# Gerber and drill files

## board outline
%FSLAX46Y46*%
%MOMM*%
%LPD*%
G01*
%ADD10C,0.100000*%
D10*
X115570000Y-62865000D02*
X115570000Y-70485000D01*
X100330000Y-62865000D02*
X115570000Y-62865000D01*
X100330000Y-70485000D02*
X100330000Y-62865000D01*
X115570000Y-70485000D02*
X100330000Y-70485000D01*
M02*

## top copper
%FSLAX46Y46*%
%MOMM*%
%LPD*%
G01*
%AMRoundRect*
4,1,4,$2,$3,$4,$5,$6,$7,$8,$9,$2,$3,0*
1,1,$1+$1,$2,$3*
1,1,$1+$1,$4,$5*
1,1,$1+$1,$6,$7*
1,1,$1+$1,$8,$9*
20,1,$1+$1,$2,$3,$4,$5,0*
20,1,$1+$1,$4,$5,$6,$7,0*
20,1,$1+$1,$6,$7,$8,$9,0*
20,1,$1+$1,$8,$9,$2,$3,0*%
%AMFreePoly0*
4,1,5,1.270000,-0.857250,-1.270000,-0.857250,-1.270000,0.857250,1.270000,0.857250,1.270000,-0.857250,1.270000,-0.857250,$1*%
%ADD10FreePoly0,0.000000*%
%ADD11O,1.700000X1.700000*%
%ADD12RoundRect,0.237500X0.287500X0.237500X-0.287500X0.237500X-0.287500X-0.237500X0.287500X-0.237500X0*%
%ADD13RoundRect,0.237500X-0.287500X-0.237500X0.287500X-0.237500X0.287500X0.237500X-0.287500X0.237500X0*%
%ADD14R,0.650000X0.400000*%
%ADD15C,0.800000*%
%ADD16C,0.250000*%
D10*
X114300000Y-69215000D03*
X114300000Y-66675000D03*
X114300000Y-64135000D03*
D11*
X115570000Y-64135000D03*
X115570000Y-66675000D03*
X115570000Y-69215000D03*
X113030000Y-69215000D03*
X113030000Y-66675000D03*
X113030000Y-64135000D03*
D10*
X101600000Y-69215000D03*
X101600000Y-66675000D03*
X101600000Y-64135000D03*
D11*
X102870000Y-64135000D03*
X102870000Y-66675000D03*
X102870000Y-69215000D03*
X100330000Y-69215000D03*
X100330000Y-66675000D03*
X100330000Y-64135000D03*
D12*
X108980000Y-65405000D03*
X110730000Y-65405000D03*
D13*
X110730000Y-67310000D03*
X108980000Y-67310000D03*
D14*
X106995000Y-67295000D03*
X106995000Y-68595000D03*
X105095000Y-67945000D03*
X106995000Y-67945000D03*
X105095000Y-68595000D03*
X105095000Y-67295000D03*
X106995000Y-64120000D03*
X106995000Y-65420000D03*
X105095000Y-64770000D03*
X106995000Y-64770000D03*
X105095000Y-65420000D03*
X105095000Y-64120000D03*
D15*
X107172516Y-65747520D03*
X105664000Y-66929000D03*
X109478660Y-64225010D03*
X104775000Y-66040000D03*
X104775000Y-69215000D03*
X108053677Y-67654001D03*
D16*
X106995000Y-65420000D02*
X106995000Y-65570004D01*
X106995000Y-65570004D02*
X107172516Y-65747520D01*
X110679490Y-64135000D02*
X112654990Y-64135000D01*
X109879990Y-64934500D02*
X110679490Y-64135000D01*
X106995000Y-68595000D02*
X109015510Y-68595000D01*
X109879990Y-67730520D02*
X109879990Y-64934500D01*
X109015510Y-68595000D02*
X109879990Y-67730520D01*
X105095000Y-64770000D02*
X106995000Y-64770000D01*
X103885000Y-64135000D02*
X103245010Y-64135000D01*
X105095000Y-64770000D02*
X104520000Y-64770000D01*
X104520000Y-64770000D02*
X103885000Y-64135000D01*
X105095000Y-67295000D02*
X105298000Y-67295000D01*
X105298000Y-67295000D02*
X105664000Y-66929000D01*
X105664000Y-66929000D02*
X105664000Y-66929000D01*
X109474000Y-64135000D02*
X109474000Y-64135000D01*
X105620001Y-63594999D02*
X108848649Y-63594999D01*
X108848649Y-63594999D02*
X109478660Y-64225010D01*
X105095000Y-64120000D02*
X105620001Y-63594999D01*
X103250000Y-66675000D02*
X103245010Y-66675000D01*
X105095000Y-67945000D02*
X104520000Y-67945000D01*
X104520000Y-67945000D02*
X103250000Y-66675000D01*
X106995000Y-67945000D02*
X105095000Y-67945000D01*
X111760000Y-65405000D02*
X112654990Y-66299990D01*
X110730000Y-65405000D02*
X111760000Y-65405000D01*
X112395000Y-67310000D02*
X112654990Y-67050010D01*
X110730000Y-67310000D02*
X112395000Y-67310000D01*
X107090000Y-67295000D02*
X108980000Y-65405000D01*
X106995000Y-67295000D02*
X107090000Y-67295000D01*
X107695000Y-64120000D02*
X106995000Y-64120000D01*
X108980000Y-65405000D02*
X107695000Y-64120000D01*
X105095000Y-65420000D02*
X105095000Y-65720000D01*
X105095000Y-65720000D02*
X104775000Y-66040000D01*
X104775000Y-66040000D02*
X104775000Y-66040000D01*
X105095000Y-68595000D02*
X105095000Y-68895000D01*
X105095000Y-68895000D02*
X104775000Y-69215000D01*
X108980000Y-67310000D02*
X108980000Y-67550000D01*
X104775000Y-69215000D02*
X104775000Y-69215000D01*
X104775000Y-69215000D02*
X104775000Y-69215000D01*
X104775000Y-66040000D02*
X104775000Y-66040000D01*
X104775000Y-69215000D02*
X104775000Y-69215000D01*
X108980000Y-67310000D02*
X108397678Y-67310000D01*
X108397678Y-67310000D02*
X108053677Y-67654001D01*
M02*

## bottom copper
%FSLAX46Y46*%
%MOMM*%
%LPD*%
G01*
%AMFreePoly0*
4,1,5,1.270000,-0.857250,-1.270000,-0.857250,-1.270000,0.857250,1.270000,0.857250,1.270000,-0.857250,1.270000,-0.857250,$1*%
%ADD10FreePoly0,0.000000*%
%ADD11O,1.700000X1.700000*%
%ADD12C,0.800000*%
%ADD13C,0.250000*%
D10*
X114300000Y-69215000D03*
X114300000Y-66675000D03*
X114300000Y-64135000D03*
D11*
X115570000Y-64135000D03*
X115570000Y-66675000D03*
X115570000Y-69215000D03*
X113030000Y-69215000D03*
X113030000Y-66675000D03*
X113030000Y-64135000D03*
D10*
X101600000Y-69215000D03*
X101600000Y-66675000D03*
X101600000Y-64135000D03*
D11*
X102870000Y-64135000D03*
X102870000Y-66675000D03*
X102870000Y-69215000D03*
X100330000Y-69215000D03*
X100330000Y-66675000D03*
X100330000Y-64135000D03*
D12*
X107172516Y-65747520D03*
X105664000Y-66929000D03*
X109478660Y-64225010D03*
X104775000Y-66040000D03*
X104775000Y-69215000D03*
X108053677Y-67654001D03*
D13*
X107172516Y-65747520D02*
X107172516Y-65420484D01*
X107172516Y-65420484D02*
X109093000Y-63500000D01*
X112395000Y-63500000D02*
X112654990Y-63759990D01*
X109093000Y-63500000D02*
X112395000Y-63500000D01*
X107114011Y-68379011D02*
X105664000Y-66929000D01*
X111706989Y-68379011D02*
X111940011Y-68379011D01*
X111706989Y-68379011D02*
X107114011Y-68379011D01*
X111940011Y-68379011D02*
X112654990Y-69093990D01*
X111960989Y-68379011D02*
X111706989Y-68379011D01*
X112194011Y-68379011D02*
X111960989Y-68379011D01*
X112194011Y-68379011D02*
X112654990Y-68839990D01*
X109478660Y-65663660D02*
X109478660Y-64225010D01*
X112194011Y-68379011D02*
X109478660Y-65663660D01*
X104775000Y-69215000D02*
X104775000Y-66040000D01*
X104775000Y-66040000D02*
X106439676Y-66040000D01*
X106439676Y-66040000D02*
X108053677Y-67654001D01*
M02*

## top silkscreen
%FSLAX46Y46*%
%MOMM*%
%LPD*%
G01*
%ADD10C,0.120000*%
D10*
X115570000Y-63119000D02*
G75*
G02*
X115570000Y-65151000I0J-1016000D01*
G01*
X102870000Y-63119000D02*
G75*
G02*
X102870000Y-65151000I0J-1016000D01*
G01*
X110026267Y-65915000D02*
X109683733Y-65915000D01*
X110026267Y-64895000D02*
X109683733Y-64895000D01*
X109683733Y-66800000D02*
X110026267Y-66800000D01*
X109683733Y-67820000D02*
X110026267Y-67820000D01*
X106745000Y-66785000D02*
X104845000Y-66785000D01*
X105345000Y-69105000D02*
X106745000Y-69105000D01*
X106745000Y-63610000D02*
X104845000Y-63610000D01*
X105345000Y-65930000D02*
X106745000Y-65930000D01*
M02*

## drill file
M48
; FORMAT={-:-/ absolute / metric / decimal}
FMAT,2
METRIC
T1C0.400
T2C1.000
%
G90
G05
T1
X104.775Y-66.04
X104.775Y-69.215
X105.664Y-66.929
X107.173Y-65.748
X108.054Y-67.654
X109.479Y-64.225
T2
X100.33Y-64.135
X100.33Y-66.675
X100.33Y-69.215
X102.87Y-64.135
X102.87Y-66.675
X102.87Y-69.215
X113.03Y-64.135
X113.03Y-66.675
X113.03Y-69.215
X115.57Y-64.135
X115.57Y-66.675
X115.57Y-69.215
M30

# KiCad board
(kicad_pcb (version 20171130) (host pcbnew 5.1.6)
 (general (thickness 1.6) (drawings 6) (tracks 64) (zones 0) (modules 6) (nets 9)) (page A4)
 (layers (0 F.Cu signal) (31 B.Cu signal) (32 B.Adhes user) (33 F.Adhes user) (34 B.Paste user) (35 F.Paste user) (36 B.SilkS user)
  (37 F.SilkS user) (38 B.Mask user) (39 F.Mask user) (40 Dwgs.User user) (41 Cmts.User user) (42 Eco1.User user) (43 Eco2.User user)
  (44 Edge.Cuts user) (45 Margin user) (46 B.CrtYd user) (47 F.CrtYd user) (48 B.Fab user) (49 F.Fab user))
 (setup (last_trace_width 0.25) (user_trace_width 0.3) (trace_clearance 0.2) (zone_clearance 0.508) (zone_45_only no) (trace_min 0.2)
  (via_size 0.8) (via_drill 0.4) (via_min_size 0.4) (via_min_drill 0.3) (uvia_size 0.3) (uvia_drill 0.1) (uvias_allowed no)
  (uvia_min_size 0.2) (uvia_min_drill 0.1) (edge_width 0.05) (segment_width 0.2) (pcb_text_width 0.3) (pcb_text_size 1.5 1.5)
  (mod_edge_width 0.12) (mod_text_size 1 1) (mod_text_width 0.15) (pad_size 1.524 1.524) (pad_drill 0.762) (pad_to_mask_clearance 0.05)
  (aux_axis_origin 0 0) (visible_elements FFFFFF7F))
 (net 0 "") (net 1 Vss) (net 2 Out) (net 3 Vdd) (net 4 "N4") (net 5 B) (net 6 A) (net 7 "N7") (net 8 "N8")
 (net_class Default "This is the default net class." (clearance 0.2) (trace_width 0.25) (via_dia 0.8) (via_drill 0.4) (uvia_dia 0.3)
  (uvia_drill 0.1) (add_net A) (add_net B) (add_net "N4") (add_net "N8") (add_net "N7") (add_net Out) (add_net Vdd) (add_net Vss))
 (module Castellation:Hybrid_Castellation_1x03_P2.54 (layer F.Cu) (at 114.3 64.135)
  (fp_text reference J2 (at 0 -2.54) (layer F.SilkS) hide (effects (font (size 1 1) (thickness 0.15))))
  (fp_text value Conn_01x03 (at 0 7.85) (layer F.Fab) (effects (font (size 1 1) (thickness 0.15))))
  (fp_arc (start 1.27 0) (end 1.27 1.016) (angle -180) (layer F.SilkS) (width 0.12))
  (pad 3 connect custom (at 0 5.08) (size 2.54 1.7145) (layers B.Cu B.Mask) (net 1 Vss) (zone_connect 0)
   (options (clearance outline) (anchor rect)) (primitives))
  (pad 2 connect custom (at 0 2.54) (size 2.54 1.7145) (layers B.Cu B.Mask) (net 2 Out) (zone_connect 0)
   (options (clearance outline) (anchor rect)) (primitives))
  (pad 1 connect custom (at 0 0) (size 2.54 1.7145) (layers B.Cu B.Mask) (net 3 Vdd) (zone_connect 0)
   (options (clearance outline) (anchor rect)) (primitives))
  (pad 3 connect custom (at 0 5.08) (size 2.54 1.7145) (layers F.Cu F.Mask) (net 1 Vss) (zone_connect 0)
   (options (clearance outline) (anchor rect)) (primitives))
  (pad 2 connect custom (at 0 2.54) (size 2.54 1.7145) (layers F.Cu F.Mask) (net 2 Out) (zone_connect 0)
   (options (clearance outline) (anchor rect)) (primitives))
  (pad 1 connect custom (at 0 0) (size 2.54 1.7145) (layers F.Cu F.Mask) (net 3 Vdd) (zone_connect 0)
   (options (clearance outline) (anchor rect)) (primitives))
  (pad 1 thru_hole oval (at 1.27 0) (size 1.7 1.7) (drill 1) (layers *.Cu *.Mask) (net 3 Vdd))
  (pad 2 thru_hole oval (at 1.27 2.54) (size 1.7 1.7) (drill 1) (layers *.Cu *.Mask) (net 2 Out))
  (pad 3 thru_hole oval (at 1.27 5.08) (size 1.7 1.7) (drill 1) (layers *.Cu *.Mask) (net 1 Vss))
  (pad 3 thru_hole oval (at -1.27 5.08) (size 1.7 1.7) (drill 1) (layers *.Cu *.Mask) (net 1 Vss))
  (pad 2 thru_hole oval (at -1.27 2.54) (size 1.7 1.7) (drill 1) (layers *.Cu *.Mask) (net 2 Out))
  (pad 1 thru_hole oval (at -1.27 0) (size 1.7 1.7) (drill 1) (layers *.Cu *.Mask) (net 3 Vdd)))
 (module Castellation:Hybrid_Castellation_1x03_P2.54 (layer F.Cu) (at 101.6 64.135)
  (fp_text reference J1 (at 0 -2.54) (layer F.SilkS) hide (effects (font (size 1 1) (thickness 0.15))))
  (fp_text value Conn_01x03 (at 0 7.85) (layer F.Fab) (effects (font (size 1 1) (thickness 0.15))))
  (fp_arc (start 1.27 0) (end 1.27 1.016) (angle -180) (layer F.SilkS) (width 0.12))
  (pad 3 connect custom (at 0 5.08) (size 2.54 1.7145) (layers B.Cu B.Mask) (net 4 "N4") (zone_connect 0)
   (options (clearance outline) (anchor rect)) (primitives))
  (pad 2 connect custom (at 0 2.54) (size 2.54 1.7145) (layers B.Cu B.Mask) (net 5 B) (zone_connect 0)
   (options (clearance outline) (anchor rect)) (primitives))
  (pad 1 connect custom (at 0 0) (size 2.54 1.7145) (layers B.Cu B.Mask) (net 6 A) (zone_connect 0)
   (options (clearance outline) (anchor rect)) (primitives))
  (pad 3 connect custom (at 0 5.08) (size 2.54 1.7145) (layers F.Cu F.Mask) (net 4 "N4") (zone_connect 0)
   (options (clearance outline) (anchor rect)) (primitives))
  (pad 2 connect custom (at 0 2.54) (size 2.54 1.7145) (layers F.Cu F.Mask) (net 5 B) (zone_connect 0)
   (options (clearance outline) (anchor rect)) (primitives))
  (pad 1 connect custom (at 0 0) (size 2.54 1.7145) (layers F.Cu F.Mask) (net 6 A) (zone_connect 0)
   (options (clearance outline) (anchor rect)) (primitives))
  (pad 1 thru_hole oval (at 1.27 0) (size 1.7 1.7) (drill 1) (layers *.Cu *.Mask) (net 6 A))
  (pad 2 thru_hole oval (at 1.27 2.54) (size 1.7 1.7) (drill 1) (layers *.Cu *.Mask) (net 5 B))
  (pad 3 thru_hole oval (at 1.27 5.08) (size 1.7 1.7) (drill 1) (layers *.Cu *.Mask) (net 4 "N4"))
  (pad 3 thru_hole oval (at -1.27 5.08) (size 1.7 1.7) (drill 1) (layers *.Cu *.Mask) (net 4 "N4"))
  (pad 2 thru_hole oval (at -1.27 2.54) (size 1.7 1.7) (drill 1) (layers *.Cu *.Mask) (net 5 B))
  (pad 1 thru_hole oval (at -1.27 0) (size 1.7 1.7) (drill 1) (layers *.Cu *.Mask) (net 6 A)))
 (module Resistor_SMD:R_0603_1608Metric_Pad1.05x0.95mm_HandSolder (layer F.Cu) (at 109.855 65.405 180)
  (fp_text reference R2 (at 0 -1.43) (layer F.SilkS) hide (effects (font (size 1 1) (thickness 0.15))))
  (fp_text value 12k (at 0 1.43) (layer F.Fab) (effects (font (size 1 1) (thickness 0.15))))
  (fp_line (start -0.171267 -0.51) (end 0.171267 -0.51) (layer F.SilkS) (width 0.12))
  (fp_line (start -0.171267 0.51) (end 0.171267 0.51) (layer F.SilkS) (width 0.12))
  (pad 2 smd roundrect (at 0.875 0 180) (size 1.05 0.95) (layers F.Cu F.Paste F.Mask) (roundrect_rratio 0.25) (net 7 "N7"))
  (pad 1 smd roundrect (at -0.875 0 180) (size 1.05 0.95) (layers F.Cu F.Paste F.Mask) (roundrect_rratio 0.25) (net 2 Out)))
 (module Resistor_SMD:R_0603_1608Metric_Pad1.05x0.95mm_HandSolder (layer F.Cu) (at 109.855 67.31)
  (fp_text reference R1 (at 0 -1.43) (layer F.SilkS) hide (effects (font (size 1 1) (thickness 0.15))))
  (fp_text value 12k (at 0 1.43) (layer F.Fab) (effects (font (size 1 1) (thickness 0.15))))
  (fp_line (start -0.171267 -0.51) (end 0.171267 -0.51) (layer F.SilkS) (width 0.12))
  (fp_line (start -0.171267 0.51) (end 0.171267 0.51) (layer F.SilkS) (width 0.12))
  (pad 2 smd roundrect (at 0.875 0) (size 1.05 0.95) (layers F.Cu F.Paste F.Mask) (roundrect_rratio 0.25) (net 2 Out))
  (pad 1 smd roundrect (at -0.875 0) (size 1.05 0.95) (layers F.Cu F.Paste F.Mask) (roundrect_rratio 0.25) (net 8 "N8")))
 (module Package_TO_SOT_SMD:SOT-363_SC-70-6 (layer F.Cu) (at 106.045 67.945)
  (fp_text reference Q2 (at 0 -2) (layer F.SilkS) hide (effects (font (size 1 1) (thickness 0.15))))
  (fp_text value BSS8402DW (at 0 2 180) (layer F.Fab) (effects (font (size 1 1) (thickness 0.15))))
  (fp_line (start 0.7 -1.16) (end -1.2 -1.16) (layer F.SilkS) (width 0.12))
  (fp_line (start -0.7 1.16) (end 0.7 1.16) (layer F.SilkS) (width 0.12))
  (pad 6 smd rect (at 0.95 -0.65) (size 0.65 0.4) (layers F.Cu F.Paste F.Mask) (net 7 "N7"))
  (pad 4 smd rect (at 0.95 0.65) (size 0.65 0.4) (layers F.Cu F.Paste F.Mask) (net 3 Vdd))
  (pad 2 smd rect (at -0.95 0) (size 0.65 0.4) (layers F.Cu F.Paste F.Mask) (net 5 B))
  (pad 5 smd rect (at 0.95 0) (size 0.65 0.4) (layers F.Cu F.Paste F.Mask) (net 5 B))
  (pad 3 smd rect (at -0.95 0.65) (size 0.65 0.4) (layers F.Cu F.Paste F.Mask) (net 8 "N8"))
  (pad 1 smd rect (at -0.95 -0.65) (size 0.65 0.4) (layers F.Cu F.Paste F.Mask) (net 1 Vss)))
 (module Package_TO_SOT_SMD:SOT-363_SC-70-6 (layer F.Cu) (at 106.045 64.77)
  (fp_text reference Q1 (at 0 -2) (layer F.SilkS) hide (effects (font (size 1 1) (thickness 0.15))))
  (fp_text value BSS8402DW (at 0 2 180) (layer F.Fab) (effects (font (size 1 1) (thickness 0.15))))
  (fp_line (start 0.7 -1.16) (end -1.2 -1.16) (layer F.SilkS) (width 0.12))
  (fp_line (start -0.7 1.16) (end 0.7 1.16) (layer F.SilkS) (width 0.12))
  (pad 6 smd rect (at 0.95 -0.65) (size 0.65 0.4) (layers F.Cu F.Paste F.Mask) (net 7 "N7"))
  (pad 4 smd rect (at 0.95 0.65) (size 0.65 0.4) (layers F.Cu F.Paste F.Mask) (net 3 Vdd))
  (pad 2 smd rect (at -0.95 0) (size 0.65 0.4) (layers F.Cu F.Paste F.Mask) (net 6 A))
  (pad 5 smd rect (at 0.95 0) (size 0.65 0.4) (layers F.Cu F.Paste F.Mask) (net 6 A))
  (pad 3 smd rect (at -0.95 0.65) (size 0.65 0.4) (layers F.Cu F.Paste F.Mask) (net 8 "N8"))
  (pad 1 smd rect (at -0.95 -0.65) (size 0.65 0.4) (layers F.Cu F.Paste F.Mask) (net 1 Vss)))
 (gr_line (start 115.57 62.865) (end 115.57 70.485) (layer Edge.Cuts) (width 0.1))
 (gr_line (start 100.33 62.865) (end 115.57 62.865) (layer Edge.Cuts) (width 0.1))
 (gr_line (start 100.33 70.485) (end 100.33 62.865) (layer Edge.Cuts) (width 0.1))
 (gr_line (start 115.57 70.485) (end 100.33 70.485) (layer Edge.Cuts) (width 0.1))
 (segment (start 106.995 65.42) (end 106.995 65.570004) (width 0.25) (layer F.Cu) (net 3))
 (via (at 107.172516 65.74752) (size 0.8) (drill 0.4) (layers F.Cu B.Cu) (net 3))
 (segment (start 106.995 65.570004) (end 107.172516 65.74752) (width 0.25) (layer F.Cu) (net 3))
 (segment (start 110.67949 64.135) (end 112.65499 64.135) (width 0.25) (layer F.Cu) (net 3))
 (segment (start 109.87999 64.9345) (end 110.67949 64.135) (width 0.25) (layer F.Cu) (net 3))
 (segment (start 106.995 68.595) (end 109.01551 68.595) (width 0.25) (layer F.Cu) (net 3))
 (segment (start 109.87999 67.73052) (end 109.87999 64.9345) (width 0.25) (layer F.Cu) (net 3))
 (segment (start 109.01551 68.595) (end 109.87999 67.73052) (width 0.25) (layer F.Cu) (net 3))
 (segment (start 107.172516 65.74752) (end 107.172516 65.420484) (width 0.25) (layer B.Cu) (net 3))
 (segment (start 107.172516 65.420484) (end 109.093 63.5) (width 0.25) (layer B.Cu) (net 3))
 (segment (start 112.395 63.5) (end 112.65499 63.75999) (width 0.25) (layer B.Cu) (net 3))
 (segment (start 109.093 63.5) (end 112.395 63.5) (width 0.25) (layer B.Cu) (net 3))
 (segment (start 105.095 64.77) (end 106.995 64.77) (width 0.25) (layer F.Cu) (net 6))
 (segment (start 103.885 64.135) (end 103.24501 64.135) (width 0.25) (layer F.Cu) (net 6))
 (segment (start 105.095 64.77) (end 104.52 64.77) (width 0.25) (layer F.Cu) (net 6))
 (segment (start 104.52 64.77) (end 103.885 64.135) (width 0.25) (layer F.Cu) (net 6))
 (segment (start 105.095 67.295) (end 105.298 67.295) (width 0.25) (layer F.Cu) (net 1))
 (segment (start 105.298 67.295) (end 105.664 66.929) (width 0.25) (layer F.Cu) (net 1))
 (segment (start 105.664 66.929) (end 105.664 66.929) (width 0.25) (layer F.Cu) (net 1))
 (via (at 105.664 66.929) (size 0.8) (drill 0.4) (layers F.Cu B.Cu) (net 1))
 (segment (start 107.114011 68.379011) (end 105.664 66.929) (width 0.25) (layer B.Cu) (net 1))
 (segment (start 111.706989 68.379011) (end 111.940011 68.379011) (width 0.25) (layer B.Cu) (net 1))
 (segment (start 111.706989 68.379011) (end 107.114011 68.379011) (width 0.25) (layer B.Cu) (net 1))
 (segment (start 111.940011 68.379011) (end 112.65499 69.09399) (width 0.25) (layer B.Cu) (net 1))
 (segment (start 109.474 64.135) (end 109.474 64.135) (width 0.25) (layer F.Cu) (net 1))
 (segment (start 111.960989 68.379011) (end 111.706989 68.379011) (width 0.25) (layer B.Cu) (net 1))
 (segment (start 112.194011 68.379011) (end 111.960989 68.379011) (width 0.25) (layer B.Cu) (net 1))
 (segment (start 112.194011 68.379011) (end 112.65499 68.83999) (width 0.25) (layer B.Cu) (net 1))
 (segment (start 105.620001 63.594999) (end 108.848649 63.594999) (width 0.25) (layer F.Cu) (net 1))
 (segment (start 108.848649 63.594999) (end 109.47866 64.22501) (width 0.25) (layer F.Cu) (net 1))
 (segment (start 109.47866 65.66366) (end 109.47866 64.22501) (width 0.25) (layer B.Cu) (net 1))
 (segment (start 112.194011 68.379011) (end 109.47866 65.66366) (width 0.25) (layer B.Cu) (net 1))
 (via (at 109.47866 64.22501) (size 0.8) (drill 0.4) (layers F.Cu B.Cu) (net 1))
 (segment (start 105.095 64.12) (end 105.620001 63.594999) (width 0.25) (layer F.Cu) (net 1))
 (segment (start 103.25 66.675) (end 103.24501 66.675) (width 0.25) (layer F.Cu) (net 5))
 (segment (start 105.095 67.945) (end 104.52 67.945) (width 0.25) (layer F.Cu) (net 5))
 (segment (start 104.52 67.945) (end 103.25 66.675) (width 0.25) (layer F.Cu) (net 5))
 (segment (start 106.995 67.945) (end 105.095 67.945) (width 0.25) (layer F.Cu) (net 5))
 (segment (start 111.76 65.405) (end 112.65499 66.29999) (width 0.25) (layer F.Cu) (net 2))
 (segment (start 110.73 65.405) (end 111.76 65.405) (width 0.25) (layer F.Cu) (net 2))
 (segment (start 112.395 67.31) (end 112.65499 67.05001) (width 0.25) (layer F.Cu) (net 2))
 (segment (start 110.73 67.31) (end 112.395 67.31) (width 0.25) (layer F.Cu) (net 2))
 (segment (start 107.09 67.295) (end 108.98 65.405) (width 0.25) (layer F.Cu) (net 7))
 (segment (start 106.995 67.295) (end 107.09 67.295) (width 0.25) (layer F.Cu) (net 7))
 (segment (start 107.695 64.12) (end 106.995 64.12) (width 0.25) (layer F.Cu) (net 7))
 (segment (start 108.98 65.405) (end 107.695 64.12) (width 0.25) (layer F.Cu) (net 7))
 (segment (start 105.095 65.42) (end 105.095 65.72) (width 0.25) (layer F.Cu) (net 8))
 (segment (start 105.095 65.72) (end 104.775 66.04) (width 0.25) (layer F.Cu) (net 8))
 (segment (start 104.775 66.04) (end 104.775 66.04) (width 0.25) (layer F.Cu) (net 8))
 (segment (start 105.095 68.595) (end 105.095 68.895) (width 0.25) (layer F.Cu) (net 8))
 (segment (start 105.095 68.895) (end 104.775 69.215) (width 0.25) (layer F.Cu) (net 8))
 (segment (start 108.98 67.31) (end 108.98 67.55) (width 0.25) (layer F.Cu) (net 8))
 (segment (start 104.775 69.215) (end 104.775 69.215) (width 0.25) (layer F.Cu) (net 8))
 (segment (start 104.775 69.215) (end 104.775 69.215) (width 0.25) (layer F.Cu) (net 8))
 (segment (start 104.775 66.04) (end 104.775 66.04) (width 0.25) (layer F.Cu) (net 8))
 (via (at 104.775 66.04) (size 0.8) (drill 0.4) (layers F.Cu B.Cu) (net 8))
 (segment (start 104.775 69.215) (end 104.775 69.215) (width 0.25) (layer F.Cu) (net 8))
 (via (at 104.775 69.215) (size 0.8) (drill 0.4) (layers F.Cu B.Cu) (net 8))
 (segment (start 104.775 69.215) (end 104.775 66.04) (width 0.25) (layer B.Cu) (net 8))
 (segment (start 108.98 67.31) (end 108.397678 67.31) (width 0.25) (layer F.Cu) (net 8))
 (segment (start 104.775 66.04) (end 106.439676 66.04) (width 0.25) (layer B.Cu) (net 8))
 (segment (start 106.439676 66.04) (end 108.053677 67.654001) (width 0.25) (layer B.Cu) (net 8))
 (via (at 108.053677 67.654001) (size 0.8) (drill 0.4) (layers F.Cu B.Cu) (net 8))
 (segment (start 108.397678 67.31) (end 108.053677 67.654001) (width 0.25) (layer F.Cu) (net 8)))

